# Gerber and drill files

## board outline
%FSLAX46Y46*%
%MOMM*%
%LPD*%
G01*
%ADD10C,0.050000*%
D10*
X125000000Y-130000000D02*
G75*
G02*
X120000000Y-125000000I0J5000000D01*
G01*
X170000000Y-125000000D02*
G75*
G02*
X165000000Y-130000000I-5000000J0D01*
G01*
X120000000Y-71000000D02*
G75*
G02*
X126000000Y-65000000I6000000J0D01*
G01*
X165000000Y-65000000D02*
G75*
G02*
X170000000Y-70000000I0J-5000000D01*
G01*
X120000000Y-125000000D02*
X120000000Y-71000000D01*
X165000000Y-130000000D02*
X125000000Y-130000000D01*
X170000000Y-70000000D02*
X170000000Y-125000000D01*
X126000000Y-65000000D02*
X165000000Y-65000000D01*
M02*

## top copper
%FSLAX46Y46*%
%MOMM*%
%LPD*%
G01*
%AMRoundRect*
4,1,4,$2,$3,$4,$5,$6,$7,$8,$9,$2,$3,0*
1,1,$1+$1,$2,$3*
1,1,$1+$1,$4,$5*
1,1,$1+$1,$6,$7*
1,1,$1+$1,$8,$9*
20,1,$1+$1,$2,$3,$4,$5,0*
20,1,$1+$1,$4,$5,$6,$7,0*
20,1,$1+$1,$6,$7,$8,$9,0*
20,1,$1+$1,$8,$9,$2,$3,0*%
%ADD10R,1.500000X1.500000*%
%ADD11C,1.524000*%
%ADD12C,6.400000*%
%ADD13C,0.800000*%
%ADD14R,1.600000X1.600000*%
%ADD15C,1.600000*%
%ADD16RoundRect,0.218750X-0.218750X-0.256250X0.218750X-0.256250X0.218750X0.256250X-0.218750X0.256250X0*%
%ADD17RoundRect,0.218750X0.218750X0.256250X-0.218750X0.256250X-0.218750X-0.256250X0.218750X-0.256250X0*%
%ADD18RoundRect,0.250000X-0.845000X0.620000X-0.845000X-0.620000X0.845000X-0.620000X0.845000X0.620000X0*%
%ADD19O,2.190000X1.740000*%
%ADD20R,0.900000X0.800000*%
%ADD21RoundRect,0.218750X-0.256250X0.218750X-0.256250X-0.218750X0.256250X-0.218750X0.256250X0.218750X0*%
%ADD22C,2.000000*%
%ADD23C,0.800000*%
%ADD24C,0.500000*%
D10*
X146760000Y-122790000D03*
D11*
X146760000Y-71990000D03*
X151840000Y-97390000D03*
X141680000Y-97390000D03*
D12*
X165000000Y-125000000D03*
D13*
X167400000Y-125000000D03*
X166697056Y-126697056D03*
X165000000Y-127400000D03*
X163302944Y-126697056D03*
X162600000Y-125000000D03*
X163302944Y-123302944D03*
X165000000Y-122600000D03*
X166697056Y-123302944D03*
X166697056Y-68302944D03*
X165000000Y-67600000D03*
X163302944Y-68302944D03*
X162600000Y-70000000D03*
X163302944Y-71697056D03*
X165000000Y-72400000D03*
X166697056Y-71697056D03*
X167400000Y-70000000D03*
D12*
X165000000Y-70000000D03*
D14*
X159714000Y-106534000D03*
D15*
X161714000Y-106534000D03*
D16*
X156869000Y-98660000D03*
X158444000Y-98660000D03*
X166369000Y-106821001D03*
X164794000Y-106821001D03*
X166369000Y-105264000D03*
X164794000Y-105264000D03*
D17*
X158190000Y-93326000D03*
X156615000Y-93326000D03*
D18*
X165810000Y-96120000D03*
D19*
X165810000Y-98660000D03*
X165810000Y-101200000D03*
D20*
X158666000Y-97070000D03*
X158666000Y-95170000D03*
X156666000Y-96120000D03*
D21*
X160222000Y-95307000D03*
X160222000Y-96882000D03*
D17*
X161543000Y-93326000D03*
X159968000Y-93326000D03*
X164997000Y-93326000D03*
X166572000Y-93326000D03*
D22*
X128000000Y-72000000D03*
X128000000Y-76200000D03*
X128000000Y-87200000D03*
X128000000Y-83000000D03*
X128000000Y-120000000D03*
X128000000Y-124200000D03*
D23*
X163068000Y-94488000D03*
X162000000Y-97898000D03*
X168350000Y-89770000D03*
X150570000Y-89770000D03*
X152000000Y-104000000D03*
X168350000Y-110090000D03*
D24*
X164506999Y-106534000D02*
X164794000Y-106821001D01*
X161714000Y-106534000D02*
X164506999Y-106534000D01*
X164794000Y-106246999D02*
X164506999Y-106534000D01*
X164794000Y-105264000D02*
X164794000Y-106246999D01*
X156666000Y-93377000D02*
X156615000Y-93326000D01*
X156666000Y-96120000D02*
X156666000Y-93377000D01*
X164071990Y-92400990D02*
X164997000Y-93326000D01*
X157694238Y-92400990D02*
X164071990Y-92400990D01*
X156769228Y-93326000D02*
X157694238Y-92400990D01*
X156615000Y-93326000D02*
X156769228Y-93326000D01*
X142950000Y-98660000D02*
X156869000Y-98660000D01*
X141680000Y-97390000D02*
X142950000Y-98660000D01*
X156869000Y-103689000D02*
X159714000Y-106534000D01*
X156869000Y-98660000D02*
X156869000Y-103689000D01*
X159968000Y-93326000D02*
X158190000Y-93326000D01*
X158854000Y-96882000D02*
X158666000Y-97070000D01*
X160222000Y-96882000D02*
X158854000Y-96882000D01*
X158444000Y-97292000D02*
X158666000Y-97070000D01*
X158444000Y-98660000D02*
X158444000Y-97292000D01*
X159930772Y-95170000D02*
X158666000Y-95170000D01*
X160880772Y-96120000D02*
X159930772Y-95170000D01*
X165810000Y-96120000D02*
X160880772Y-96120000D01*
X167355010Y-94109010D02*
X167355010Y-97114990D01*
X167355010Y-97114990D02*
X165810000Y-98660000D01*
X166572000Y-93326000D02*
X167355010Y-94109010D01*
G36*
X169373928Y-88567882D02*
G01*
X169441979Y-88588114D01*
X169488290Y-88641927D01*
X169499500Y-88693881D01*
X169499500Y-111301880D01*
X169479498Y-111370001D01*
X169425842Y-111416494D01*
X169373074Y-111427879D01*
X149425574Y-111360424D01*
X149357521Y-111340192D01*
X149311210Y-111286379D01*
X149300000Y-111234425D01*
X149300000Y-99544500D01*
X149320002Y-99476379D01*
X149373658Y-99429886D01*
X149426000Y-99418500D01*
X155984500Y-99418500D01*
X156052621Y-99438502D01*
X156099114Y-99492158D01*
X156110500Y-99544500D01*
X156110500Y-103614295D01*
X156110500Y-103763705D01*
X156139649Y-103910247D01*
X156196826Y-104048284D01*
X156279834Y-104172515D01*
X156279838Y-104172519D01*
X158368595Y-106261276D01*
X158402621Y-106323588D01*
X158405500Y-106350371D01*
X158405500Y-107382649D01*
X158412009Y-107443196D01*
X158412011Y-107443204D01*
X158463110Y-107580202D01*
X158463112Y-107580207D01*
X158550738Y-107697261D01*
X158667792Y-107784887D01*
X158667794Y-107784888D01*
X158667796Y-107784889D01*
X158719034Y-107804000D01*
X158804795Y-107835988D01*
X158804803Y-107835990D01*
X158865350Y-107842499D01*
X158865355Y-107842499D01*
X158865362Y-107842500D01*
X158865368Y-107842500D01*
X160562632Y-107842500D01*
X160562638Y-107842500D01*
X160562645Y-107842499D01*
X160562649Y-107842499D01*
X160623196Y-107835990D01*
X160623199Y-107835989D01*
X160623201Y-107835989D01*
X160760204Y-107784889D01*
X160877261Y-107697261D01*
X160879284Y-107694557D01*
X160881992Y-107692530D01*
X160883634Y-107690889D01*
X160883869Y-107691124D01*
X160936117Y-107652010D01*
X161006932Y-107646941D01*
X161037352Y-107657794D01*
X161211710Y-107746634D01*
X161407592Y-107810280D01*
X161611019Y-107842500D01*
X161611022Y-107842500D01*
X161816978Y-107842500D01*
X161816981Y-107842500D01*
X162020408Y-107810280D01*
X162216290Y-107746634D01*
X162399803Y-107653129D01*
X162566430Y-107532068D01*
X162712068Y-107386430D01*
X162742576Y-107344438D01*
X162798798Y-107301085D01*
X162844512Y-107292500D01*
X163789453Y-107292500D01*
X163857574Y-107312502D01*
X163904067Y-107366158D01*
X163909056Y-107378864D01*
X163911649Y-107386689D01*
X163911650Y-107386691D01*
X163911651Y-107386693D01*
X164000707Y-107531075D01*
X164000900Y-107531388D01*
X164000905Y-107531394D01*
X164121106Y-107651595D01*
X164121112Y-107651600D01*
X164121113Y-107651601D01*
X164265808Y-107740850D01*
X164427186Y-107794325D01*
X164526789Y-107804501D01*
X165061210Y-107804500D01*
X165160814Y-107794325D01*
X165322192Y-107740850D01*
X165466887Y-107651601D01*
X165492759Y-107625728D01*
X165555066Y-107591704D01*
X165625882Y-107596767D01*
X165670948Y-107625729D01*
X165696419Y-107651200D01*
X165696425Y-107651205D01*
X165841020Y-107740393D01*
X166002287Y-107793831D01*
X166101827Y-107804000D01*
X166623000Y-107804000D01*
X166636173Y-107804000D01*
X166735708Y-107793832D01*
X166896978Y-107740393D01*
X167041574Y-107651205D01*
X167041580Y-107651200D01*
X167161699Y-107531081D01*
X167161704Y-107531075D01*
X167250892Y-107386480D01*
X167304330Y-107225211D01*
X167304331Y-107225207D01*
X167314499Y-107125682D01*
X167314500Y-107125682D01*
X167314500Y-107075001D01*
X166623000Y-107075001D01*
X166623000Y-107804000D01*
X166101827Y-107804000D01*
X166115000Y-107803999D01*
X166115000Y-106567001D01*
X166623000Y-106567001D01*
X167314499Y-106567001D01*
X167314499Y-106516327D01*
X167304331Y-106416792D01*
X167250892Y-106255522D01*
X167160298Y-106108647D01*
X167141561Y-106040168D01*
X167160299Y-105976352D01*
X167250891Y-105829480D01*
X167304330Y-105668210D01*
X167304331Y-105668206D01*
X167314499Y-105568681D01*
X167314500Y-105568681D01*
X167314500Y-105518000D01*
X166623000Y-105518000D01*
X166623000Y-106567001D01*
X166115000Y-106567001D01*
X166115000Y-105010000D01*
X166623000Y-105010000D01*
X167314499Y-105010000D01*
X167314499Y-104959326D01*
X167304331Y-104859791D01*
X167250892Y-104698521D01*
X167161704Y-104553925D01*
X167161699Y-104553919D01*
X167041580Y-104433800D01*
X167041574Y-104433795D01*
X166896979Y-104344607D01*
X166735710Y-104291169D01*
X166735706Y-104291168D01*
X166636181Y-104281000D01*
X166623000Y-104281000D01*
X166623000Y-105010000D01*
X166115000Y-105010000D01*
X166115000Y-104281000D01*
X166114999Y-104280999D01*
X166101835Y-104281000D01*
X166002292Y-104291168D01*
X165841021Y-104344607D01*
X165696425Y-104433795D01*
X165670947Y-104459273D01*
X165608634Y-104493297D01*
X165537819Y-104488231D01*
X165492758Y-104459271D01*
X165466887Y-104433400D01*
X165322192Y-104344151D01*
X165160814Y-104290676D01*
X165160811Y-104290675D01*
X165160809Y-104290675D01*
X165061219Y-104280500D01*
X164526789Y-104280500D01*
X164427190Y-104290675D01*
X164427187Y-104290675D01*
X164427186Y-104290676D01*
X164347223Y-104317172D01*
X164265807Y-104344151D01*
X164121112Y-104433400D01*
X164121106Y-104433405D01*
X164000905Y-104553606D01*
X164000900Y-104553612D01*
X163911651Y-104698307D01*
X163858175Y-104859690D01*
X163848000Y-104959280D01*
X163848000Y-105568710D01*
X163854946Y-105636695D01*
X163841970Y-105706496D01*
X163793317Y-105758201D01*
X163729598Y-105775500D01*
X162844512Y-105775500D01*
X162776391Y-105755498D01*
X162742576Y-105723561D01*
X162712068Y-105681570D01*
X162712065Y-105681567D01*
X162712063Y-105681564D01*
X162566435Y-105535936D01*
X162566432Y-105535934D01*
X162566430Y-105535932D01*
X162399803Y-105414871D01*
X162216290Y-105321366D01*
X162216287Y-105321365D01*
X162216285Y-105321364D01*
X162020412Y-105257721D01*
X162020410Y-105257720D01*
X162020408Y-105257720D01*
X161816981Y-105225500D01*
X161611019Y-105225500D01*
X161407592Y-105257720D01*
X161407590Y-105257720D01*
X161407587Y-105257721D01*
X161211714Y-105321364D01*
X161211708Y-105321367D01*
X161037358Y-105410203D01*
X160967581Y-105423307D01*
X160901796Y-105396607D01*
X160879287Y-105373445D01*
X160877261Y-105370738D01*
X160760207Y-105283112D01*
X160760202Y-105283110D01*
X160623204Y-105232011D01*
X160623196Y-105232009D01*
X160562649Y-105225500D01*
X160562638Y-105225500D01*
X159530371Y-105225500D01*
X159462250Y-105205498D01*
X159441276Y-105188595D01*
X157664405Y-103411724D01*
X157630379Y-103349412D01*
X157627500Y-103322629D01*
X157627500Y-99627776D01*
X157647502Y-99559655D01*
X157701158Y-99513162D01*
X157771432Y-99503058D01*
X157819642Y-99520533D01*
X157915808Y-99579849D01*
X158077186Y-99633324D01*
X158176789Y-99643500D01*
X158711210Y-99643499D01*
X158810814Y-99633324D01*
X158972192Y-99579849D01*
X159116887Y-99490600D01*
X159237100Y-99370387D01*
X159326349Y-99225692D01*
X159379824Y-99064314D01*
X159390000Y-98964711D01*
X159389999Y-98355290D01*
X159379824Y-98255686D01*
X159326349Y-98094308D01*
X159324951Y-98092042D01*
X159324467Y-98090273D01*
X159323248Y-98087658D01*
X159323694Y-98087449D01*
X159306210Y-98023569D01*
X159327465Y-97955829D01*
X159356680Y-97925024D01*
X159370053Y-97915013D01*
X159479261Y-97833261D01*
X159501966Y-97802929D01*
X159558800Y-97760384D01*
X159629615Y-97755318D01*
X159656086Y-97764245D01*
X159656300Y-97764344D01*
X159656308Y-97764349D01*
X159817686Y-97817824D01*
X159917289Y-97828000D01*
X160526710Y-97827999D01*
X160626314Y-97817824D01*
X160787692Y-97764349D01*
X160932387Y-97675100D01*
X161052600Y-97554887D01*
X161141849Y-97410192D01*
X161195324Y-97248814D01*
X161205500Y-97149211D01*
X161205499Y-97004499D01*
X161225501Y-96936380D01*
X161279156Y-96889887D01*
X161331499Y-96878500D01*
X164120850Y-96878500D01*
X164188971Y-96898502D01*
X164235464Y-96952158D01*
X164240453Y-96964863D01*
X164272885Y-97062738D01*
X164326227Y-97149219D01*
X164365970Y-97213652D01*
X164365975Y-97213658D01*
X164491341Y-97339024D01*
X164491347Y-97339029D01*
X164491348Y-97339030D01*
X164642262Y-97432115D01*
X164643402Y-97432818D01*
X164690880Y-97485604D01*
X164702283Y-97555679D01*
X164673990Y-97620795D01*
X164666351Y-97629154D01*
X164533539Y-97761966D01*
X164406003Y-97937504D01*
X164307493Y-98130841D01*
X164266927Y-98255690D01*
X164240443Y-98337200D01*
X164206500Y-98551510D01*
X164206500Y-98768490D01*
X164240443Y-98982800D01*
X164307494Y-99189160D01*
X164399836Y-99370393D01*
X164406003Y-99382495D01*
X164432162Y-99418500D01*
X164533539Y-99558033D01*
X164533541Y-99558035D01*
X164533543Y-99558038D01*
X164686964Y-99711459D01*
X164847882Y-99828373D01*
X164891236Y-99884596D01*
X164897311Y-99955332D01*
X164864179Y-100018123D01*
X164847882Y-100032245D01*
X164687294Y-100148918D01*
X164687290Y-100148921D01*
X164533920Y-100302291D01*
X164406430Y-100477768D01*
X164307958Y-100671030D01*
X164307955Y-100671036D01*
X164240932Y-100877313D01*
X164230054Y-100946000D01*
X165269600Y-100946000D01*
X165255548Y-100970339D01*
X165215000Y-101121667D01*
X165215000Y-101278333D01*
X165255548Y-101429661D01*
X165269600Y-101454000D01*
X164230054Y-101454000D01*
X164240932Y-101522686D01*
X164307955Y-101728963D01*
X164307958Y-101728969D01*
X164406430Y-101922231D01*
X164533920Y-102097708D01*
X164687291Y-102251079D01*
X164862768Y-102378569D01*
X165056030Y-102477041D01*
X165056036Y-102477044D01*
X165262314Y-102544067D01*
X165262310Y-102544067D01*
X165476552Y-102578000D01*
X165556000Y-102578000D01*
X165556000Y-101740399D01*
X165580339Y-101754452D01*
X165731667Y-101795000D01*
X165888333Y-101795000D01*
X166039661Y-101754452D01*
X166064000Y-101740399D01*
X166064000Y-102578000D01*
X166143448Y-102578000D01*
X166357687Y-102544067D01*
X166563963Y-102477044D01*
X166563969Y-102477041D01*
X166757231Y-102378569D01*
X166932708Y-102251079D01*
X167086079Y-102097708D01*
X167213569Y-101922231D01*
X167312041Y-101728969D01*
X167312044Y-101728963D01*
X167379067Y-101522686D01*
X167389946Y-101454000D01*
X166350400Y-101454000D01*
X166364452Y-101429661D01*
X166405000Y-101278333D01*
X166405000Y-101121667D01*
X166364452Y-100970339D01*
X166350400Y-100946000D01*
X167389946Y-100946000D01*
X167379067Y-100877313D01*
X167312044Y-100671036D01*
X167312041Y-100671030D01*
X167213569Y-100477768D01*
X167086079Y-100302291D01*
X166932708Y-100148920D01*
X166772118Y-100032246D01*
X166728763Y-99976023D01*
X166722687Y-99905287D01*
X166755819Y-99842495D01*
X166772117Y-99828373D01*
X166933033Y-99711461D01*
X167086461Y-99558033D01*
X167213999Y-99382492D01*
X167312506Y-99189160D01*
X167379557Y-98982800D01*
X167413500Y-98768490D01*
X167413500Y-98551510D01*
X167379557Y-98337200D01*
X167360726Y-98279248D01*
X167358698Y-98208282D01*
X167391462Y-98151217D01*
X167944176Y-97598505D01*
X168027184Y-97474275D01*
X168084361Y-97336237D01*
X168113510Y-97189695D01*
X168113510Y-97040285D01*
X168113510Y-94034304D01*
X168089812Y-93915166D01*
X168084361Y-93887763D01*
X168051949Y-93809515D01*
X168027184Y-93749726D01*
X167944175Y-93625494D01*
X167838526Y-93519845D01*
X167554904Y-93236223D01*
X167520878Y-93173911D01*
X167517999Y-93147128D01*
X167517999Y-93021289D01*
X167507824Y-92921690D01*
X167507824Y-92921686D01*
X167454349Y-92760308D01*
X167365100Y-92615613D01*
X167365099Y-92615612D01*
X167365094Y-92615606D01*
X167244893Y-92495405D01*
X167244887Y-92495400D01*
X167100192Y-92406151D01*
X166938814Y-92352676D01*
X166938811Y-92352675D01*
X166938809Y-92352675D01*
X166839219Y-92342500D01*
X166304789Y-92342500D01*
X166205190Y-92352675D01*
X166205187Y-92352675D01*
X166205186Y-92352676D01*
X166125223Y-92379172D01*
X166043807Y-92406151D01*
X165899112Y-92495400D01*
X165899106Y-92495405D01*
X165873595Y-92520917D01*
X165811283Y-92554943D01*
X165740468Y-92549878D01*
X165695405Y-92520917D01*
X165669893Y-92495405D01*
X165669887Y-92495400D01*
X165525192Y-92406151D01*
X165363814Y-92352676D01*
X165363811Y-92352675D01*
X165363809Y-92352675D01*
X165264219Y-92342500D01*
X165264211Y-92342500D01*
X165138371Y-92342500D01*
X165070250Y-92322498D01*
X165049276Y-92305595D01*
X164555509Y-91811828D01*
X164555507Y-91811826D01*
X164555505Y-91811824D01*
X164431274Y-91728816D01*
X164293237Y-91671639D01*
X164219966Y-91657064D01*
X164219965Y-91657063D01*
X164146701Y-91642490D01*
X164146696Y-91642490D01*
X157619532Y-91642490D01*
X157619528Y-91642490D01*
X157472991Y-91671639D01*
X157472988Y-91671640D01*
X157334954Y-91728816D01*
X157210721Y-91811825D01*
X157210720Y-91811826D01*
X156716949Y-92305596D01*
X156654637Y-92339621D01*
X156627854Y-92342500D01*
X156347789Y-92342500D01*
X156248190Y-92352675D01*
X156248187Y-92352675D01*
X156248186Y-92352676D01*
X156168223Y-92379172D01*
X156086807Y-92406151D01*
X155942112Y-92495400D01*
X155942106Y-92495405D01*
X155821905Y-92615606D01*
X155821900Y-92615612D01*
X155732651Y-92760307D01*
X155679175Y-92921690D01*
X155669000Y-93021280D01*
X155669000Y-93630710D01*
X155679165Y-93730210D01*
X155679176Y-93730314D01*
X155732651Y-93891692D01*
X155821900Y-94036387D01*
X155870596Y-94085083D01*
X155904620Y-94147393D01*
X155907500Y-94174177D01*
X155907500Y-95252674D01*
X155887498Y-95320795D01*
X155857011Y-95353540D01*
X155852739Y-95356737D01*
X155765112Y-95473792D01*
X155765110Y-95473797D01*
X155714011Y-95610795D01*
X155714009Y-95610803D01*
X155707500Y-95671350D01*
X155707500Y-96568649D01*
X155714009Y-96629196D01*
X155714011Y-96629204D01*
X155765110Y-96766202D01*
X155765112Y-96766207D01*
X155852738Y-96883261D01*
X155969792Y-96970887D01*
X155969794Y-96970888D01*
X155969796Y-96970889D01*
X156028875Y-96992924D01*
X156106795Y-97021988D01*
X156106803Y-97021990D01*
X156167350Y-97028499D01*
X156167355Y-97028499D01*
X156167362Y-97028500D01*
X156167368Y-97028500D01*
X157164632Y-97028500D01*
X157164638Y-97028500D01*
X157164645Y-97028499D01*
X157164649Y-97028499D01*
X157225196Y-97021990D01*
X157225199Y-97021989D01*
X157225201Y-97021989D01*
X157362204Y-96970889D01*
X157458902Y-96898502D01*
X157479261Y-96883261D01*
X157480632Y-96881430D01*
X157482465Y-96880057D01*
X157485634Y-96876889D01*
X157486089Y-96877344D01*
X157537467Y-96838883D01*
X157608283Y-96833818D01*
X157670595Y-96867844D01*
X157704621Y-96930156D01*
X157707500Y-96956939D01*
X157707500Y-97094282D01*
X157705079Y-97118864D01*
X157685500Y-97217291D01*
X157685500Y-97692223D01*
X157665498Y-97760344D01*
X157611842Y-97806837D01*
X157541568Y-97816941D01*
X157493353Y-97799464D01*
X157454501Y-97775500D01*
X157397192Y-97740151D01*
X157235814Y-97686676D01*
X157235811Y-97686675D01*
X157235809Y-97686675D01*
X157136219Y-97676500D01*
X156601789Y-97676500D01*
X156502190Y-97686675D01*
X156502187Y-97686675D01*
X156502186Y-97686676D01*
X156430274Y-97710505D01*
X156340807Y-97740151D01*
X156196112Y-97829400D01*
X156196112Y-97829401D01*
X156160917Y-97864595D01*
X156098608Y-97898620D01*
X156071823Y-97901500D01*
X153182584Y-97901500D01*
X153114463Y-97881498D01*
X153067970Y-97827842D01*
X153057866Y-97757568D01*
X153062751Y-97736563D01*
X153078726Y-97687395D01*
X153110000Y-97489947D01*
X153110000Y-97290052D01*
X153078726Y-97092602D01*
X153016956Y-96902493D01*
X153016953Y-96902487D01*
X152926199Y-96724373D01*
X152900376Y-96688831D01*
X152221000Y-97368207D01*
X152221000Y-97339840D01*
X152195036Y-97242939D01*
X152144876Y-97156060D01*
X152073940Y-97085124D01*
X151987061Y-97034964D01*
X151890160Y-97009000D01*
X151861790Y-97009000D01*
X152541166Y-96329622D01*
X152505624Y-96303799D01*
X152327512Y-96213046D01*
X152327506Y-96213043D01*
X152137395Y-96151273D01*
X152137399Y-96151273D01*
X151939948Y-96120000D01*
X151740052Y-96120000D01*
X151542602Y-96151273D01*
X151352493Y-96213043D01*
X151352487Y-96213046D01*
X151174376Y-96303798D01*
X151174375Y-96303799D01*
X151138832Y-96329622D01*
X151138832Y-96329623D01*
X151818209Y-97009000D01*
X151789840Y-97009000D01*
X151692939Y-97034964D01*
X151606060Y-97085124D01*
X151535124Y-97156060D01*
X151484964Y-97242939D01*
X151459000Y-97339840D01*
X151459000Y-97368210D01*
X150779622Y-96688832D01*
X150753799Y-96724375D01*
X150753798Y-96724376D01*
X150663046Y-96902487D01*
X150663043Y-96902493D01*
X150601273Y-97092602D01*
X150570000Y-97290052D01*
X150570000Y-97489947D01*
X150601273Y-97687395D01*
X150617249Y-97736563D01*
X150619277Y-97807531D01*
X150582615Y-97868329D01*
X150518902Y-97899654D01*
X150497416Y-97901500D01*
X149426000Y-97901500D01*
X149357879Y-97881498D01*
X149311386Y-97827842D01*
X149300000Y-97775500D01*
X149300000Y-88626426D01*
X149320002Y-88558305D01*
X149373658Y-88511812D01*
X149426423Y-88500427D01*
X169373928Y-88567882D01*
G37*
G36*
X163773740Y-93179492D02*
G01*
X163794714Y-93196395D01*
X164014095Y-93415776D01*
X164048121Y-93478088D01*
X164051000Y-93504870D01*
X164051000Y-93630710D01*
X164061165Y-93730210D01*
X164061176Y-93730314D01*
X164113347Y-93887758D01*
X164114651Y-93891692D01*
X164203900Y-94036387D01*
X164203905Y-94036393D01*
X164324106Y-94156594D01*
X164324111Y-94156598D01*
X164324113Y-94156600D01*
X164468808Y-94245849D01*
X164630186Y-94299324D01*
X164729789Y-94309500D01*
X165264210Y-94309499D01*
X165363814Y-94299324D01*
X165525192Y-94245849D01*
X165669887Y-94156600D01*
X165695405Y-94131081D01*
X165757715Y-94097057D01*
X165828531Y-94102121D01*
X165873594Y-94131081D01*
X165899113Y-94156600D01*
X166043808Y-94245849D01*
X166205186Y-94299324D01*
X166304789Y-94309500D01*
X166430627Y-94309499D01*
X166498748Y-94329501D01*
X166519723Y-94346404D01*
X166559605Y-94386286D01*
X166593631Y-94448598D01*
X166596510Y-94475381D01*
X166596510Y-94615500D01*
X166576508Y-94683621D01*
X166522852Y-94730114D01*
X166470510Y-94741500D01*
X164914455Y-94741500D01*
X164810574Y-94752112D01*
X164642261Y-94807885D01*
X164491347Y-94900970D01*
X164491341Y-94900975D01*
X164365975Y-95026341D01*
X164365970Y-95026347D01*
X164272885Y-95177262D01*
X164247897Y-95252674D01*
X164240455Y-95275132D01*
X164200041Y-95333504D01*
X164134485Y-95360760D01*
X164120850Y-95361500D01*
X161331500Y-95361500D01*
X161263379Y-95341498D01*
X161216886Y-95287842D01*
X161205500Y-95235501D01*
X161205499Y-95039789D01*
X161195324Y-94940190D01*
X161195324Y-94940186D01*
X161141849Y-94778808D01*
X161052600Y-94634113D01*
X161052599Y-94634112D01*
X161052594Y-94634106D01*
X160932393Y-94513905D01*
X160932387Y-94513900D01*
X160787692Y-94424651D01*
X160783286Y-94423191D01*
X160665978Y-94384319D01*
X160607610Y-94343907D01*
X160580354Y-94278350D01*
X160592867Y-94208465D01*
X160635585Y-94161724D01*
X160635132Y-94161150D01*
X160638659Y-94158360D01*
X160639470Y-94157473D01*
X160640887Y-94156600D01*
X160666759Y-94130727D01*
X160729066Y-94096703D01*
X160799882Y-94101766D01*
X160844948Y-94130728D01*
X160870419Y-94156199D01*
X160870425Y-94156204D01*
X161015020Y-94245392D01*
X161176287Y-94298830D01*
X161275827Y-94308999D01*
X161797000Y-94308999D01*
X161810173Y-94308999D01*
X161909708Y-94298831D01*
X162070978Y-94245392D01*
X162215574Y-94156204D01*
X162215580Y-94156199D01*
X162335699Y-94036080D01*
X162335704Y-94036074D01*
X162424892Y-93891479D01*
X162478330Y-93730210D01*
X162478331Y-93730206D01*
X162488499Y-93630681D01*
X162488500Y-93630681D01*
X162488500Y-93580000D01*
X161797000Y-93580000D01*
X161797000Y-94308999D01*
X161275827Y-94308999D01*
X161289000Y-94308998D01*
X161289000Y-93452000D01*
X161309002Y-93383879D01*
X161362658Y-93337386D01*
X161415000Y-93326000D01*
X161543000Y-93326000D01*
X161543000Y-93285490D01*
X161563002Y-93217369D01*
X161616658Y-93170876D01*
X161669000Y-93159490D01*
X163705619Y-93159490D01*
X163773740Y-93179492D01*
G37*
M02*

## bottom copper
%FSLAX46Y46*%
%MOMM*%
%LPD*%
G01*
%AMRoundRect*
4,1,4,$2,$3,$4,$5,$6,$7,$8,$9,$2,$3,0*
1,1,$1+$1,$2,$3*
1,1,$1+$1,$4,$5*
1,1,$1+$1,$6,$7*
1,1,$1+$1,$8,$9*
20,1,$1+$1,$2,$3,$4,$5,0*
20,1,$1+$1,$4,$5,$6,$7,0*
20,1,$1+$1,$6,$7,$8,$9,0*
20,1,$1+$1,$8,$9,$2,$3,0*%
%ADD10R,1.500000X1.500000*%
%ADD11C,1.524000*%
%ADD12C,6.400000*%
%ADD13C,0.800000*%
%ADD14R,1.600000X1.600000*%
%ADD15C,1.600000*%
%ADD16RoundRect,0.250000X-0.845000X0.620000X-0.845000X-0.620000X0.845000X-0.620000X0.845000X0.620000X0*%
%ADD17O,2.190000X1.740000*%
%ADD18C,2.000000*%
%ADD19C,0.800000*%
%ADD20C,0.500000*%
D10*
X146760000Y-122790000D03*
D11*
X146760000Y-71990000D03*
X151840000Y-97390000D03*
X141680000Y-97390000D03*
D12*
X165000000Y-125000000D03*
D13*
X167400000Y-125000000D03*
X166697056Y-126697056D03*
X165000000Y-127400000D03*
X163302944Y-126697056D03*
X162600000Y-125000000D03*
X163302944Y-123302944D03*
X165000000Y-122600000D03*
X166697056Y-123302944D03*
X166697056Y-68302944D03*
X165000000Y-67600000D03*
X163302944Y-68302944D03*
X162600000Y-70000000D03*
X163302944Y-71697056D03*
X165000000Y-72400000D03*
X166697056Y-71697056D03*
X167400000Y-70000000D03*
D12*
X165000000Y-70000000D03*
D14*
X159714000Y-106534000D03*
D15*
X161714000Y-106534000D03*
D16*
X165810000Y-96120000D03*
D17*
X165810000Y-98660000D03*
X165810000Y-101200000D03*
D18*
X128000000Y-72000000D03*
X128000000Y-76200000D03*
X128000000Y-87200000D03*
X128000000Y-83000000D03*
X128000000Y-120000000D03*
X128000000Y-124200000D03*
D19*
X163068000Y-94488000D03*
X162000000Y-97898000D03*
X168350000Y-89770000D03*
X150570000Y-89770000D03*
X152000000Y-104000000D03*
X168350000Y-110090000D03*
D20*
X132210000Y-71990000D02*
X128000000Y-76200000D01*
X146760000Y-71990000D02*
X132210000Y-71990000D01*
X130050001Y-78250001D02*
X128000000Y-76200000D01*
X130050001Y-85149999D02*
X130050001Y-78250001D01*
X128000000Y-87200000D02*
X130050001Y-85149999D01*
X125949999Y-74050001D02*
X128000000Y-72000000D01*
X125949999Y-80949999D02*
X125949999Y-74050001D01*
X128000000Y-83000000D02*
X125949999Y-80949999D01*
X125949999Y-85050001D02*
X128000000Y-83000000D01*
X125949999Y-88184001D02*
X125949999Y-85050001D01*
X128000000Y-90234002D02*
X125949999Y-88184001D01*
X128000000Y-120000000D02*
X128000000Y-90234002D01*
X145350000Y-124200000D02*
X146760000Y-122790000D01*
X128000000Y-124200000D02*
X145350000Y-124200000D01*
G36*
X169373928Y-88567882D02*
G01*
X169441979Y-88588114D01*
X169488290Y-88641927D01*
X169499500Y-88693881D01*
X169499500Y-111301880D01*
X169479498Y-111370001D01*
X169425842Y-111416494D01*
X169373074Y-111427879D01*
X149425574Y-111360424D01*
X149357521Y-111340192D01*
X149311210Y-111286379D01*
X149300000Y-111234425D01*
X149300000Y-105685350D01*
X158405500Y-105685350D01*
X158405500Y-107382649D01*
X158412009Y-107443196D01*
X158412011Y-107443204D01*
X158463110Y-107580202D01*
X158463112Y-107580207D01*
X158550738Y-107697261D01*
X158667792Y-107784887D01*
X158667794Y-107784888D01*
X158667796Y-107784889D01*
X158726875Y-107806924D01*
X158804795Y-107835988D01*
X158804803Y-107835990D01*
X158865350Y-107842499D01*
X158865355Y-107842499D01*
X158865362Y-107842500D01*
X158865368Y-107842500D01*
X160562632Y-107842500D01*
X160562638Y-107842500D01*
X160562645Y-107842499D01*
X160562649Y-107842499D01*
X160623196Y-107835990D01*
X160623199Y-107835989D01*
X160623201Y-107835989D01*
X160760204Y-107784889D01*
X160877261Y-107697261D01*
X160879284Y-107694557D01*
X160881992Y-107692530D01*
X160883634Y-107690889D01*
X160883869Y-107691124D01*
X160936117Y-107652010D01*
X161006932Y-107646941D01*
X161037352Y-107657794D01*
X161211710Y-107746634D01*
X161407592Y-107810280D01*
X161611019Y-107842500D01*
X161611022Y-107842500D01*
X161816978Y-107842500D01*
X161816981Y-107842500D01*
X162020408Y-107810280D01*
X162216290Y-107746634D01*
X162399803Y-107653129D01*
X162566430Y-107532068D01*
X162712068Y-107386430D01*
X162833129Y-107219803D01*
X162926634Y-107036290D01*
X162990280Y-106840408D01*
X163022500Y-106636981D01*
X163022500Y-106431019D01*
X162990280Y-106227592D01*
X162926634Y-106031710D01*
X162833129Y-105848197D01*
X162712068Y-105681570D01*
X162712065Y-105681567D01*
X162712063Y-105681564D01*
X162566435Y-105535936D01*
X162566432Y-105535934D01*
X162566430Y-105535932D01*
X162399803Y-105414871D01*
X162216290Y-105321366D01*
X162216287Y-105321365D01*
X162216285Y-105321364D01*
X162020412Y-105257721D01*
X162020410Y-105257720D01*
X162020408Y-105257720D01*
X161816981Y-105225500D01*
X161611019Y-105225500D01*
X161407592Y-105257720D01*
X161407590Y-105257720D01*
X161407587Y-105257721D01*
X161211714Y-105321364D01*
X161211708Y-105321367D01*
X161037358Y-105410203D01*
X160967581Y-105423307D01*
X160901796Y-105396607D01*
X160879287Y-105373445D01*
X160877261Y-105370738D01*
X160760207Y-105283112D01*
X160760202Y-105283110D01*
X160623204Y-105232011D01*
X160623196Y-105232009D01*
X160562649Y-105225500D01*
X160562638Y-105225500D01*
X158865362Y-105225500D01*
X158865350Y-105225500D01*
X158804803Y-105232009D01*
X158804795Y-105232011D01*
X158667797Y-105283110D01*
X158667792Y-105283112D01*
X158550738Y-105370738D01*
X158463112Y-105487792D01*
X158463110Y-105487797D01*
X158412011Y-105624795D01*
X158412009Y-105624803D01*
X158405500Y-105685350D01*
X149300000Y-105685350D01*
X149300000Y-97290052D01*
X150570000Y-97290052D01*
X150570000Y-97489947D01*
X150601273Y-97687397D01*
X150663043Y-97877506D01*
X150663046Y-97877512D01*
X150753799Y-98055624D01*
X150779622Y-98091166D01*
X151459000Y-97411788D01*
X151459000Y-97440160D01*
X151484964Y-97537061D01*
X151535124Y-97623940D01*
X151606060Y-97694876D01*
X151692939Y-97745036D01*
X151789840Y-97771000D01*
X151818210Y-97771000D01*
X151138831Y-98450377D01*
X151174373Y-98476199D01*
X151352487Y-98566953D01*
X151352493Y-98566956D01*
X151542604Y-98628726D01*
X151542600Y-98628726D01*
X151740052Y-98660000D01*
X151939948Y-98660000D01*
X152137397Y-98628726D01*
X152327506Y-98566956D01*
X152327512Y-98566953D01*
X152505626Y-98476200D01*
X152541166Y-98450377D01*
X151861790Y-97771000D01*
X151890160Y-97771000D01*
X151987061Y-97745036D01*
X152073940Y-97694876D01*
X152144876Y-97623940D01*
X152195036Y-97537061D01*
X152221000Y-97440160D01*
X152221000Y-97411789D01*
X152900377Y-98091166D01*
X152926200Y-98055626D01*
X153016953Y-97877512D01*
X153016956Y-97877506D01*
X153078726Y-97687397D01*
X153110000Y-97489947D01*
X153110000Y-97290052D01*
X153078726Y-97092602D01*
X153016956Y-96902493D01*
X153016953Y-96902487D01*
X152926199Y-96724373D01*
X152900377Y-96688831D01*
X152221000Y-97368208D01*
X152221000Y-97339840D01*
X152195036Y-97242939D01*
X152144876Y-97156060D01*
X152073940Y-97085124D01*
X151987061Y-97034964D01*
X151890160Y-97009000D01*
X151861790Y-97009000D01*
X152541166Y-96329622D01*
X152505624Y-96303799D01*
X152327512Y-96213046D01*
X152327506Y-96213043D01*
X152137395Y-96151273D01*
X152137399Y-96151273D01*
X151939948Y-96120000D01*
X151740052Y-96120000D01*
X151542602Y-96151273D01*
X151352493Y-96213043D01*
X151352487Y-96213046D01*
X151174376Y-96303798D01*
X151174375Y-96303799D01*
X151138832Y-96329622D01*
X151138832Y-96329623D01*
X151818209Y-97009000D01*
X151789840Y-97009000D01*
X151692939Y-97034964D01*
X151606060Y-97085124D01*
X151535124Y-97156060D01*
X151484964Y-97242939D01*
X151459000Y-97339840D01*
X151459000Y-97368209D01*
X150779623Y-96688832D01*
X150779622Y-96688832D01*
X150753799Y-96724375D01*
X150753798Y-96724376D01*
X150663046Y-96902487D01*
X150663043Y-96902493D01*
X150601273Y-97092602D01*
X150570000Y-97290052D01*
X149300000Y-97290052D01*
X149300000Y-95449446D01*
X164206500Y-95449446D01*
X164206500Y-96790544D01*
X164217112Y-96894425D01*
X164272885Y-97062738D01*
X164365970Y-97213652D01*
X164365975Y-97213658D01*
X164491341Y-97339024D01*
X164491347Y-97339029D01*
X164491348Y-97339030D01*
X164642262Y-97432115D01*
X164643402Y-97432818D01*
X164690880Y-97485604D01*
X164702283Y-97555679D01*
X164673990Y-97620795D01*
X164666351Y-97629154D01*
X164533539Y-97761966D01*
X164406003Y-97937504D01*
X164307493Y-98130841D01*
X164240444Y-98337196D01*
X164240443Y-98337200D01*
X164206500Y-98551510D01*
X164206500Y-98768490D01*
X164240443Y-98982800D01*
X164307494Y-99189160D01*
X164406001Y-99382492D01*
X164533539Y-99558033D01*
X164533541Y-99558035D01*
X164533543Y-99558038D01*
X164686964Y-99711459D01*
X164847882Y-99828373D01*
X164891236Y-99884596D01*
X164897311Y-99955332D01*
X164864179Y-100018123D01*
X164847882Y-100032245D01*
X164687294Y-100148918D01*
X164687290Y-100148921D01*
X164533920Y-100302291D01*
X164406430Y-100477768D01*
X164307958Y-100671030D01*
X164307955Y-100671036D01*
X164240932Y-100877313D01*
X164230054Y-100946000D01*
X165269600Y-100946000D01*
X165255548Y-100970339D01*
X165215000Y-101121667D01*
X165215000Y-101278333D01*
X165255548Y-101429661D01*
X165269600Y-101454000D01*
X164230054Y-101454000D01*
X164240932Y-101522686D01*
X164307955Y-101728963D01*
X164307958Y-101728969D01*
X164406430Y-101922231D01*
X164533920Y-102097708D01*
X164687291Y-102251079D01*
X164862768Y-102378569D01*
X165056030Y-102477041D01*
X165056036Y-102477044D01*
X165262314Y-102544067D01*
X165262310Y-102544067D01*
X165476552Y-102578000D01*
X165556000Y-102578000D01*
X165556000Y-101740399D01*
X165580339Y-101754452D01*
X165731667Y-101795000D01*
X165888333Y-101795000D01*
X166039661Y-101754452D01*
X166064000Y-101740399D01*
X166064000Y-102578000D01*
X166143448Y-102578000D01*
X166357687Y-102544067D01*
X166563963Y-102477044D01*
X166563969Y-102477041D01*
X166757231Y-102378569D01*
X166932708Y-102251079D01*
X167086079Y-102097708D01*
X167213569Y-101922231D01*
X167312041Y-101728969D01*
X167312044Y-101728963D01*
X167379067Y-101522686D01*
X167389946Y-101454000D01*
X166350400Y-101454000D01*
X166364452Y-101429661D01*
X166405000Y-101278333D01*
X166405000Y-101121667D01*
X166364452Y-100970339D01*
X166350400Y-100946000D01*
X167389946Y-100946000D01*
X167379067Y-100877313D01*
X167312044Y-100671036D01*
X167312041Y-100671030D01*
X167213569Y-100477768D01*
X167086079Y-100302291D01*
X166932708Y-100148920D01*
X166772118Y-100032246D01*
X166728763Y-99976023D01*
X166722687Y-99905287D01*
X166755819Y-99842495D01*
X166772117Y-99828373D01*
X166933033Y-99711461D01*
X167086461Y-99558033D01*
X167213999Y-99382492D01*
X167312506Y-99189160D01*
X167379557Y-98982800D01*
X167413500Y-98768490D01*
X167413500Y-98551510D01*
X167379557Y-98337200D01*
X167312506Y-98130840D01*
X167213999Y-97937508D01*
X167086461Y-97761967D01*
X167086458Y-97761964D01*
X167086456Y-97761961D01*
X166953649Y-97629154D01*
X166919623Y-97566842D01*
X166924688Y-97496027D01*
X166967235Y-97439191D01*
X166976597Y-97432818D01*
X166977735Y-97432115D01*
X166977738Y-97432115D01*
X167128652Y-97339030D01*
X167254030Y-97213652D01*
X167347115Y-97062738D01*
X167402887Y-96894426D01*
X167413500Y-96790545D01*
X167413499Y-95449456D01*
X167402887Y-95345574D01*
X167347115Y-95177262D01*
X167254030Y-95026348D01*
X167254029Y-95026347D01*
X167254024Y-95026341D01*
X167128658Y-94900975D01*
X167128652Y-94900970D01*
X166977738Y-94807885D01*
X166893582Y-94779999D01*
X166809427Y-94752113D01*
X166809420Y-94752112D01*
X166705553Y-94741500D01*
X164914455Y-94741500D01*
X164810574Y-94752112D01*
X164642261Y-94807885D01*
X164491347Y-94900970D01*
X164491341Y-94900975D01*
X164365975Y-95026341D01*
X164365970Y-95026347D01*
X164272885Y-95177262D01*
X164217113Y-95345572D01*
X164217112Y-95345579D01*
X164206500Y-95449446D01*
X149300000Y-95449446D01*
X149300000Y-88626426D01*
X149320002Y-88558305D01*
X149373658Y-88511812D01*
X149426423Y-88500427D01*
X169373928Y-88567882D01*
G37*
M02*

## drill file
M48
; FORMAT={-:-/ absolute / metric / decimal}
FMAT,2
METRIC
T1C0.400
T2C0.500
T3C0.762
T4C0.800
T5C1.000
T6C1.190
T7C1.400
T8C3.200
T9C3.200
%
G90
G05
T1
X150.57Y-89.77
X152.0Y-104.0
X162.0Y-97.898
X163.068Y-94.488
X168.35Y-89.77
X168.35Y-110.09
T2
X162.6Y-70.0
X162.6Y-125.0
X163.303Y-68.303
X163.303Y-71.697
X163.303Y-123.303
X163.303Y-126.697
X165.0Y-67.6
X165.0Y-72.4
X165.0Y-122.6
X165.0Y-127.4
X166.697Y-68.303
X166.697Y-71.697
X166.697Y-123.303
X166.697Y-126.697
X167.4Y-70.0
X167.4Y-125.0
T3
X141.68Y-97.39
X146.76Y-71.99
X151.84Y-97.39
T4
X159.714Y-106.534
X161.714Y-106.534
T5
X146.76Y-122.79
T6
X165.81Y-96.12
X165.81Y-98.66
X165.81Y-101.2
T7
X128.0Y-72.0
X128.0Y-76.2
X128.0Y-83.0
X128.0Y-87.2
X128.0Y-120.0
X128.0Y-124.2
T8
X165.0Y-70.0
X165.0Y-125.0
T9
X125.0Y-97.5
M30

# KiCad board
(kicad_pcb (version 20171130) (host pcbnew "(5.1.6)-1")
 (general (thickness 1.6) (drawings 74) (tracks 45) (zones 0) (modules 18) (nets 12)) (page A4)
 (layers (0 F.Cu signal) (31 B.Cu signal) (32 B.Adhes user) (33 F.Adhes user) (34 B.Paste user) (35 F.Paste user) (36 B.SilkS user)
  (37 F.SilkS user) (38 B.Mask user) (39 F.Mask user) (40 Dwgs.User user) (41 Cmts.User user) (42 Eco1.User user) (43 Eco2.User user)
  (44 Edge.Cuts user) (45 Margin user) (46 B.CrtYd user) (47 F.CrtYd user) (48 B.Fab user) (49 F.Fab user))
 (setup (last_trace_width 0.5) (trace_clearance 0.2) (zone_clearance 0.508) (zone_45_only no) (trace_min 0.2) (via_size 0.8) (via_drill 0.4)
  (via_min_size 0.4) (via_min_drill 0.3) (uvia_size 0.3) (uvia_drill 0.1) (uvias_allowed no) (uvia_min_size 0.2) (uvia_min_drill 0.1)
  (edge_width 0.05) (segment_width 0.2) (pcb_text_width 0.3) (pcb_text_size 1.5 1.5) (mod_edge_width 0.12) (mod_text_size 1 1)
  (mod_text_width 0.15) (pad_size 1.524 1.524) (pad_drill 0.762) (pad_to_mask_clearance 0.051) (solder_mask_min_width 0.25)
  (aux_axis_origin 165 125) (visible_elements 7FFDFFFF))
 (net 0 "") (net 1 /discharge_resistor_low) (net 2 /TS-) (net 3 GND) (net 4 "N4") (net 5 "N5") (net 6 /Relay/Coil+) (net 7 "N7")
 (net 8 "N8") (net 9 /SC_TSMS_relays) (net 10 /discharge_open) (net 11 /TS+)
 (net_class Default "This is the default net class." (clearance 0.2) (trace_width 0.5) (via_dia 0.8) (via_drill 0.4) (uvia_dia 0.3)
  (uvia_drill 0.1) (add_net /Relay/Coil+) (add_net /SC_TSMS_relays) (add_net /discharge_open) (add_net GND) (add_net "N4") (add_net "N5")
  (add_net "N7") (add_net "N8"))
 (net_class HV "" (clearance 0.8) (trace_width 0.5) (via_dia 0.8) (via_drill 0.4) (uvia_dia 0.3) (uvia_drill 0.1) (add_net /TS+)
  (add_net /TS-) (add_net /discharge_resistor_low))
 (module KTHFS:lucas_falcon (layer F.Cu) (at 165 79)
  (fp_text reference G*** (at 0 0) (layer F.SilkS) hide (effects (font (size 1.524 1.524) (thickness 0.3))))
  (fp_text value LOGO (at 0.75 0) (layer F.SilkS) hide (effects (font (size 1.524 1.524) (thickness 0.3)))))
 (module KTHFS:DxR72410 (layer F.Cu) (at 146.76 122.79 90)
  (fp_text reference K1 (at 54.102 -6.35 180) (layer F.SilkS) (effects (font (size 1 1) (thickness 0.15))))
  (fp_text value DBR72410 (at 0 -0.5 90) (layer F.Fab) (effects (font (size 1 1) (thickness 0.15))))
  (pad 1 thru_hole rect (at 0 0 90) (size 1.5 1.5) (drill 1) (layers *.Cu *.Mask) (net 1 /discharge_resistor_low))
  (pad 2 thru_hole circle (at 50.8 0 90) (size 1.524 1.524) (drill 0.762) (layers *.Cu *.Mask) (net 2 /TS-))
  (pad 3 thru_hole circle (at 25.4 5.08 90) (size 1.524 1.524) (drill 0.762) (layers *.Cu *.Mask) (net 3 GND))
  (pad 4 thru_hole circle (at 25.4 -5.08 90) (size 1.524 1.524) (drill 0.762) (layers *.Cu *.Mask) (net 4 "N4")))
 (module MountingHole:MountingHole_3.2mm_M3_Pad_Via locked (layer F.Cu) (at 165 125)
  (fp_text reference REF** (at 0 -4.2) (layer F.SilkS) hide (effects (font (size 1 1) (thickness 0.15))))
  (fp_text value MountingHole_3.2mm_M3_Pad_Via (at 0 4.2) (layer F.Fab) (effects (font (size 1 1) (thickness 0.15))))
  (pad 1 thru_hole circle (at 0 0) (size 6.4 6.4) (drill 3.2) (layers *.Cu *.Mask))
  (pad 1 thru_hole circle (at 2.4 0) (size 0.8 0.8) (drill 0.5) (layers *.Cu *.Mask))
  (pad 1 thru_hole circle (at 1.697056 1.697056) (size 0.8 0.8) (drill 0.5) (layers *.Cu *.Mask))
  (pad 1 thru_hole circle (at 0 2.4) (size 0.8 0.8) (drill 0.5) (layers *.Cu *.Mask))
  (pad 1 thru_hole circle (at -1.697056 1.697056) (size 0.8 0.8) (drill 0.5) (layers *.Cu *.Mask))
  (pad 1 thru_hole circle (at -2.4 0) (size 0.8 0.8) (drill 0.5) (layers *.Cu *.Mask))
  (pad 1 thru_hole circle (at -1.697056 -1.697056) (size 0.8 0.8) (drill 0.5) (layers *.Cu *.Mask))
  (pad 1 thru_hole circle (at 0 -2.4) (size 0.8 0.8) (drill 0.5) (layers *.Cu *.Mask))
  (pad 1 thru_hole circle (at 1.697056 -1.697056) (size 0.8 0.8) (drill 0.5) (layers *.Cu *.Mask)))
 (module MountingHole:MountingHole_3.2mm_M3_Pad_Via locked (layer F.Cu) (at 165 70)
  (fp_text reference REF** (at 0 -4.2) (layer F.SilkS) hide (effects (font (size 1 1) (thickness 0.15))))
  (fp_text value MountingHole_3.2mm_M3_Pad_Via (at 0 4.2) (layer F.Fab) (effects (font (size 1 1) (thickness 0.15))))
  (pad 1 thru_hole circle (at 1.697056 -1.697056) (size 0.8 0.8) (drill 0.5) (layers *.Cu *.Mask))
  (pad 1 thru_hole circle (at 0 -2.4) (size 0.8 0.8) (drill 0.5) (layers *.Cu *.Mask))
  (pad 1 thru_hole circle (at -1.697056 -1.697056) (size 0.8 0.8) (drill 0.5) (layers *.Cu *.Mask))
  (pad 1 thru_hole circle (at -2.4 0) (size 0.8 0.8) (drill 0.5) (layers *.Cu *.Mask))
  (pad 1 thru_hole circle (at -1.697056 1.697056) (size 0.8 0.8) (drill 0.5) (layers *.Cu *.Mask))
  (pad 1 thru_hole circle (at 0 2.4) (size 0.8 0.8) (drill 0.5) (layers *.Cu *.Mask))
  (pad 1 thru_hole circle (at 1.697056 1.697056) (size 0.8 0.8) (drill 0.5) (layers *.Cu *.Mask))
  (pad 1 thru_hole circle (at 2.4 0) (size 0.8 0.8) (drill 0.5) (layers *.Cu *.Mask))
  (pad 1 thru_hole circle (at 0 0) (size 6.4 6.4) (drill 3.2) (layers *.Cu *.Mask)))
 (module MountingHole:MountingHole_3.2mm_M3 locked (layer F.Cu) (at 125 97.5)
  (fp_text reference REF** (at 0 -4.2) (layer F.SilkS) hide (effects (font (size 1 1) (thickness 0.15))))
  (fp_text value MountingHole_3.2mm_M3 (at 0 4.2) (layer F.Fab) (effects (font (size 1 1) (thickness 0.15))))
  (pad 1 np_thru_hole circle (at 0 0) (size 3.2 3.2) (drill 3.2) (layers *.Cu *.Mask)))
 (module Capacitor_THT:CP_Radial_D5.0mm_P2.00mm (layer F.Cu) (at 159.714 106.534)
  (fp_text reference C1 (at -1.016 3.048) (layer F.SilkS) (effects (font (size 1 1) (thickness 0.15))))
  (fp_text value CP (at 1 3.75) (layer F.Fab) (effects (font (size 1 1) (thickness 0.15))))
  (pad 1 thru_hole rect (at 0 0) (size 1.6 1.6) (drill 0.8) (layers *.Cu *.Mask) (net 4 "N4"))
  (pad 2 thru_hole circle (at 2 0) (size 1.6 1.6) (drill 0.8) (layers *.Cu *.Mask) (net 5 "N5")))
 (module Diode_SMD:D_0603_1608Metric (layer F.Cu) (at 157.6565 98.66)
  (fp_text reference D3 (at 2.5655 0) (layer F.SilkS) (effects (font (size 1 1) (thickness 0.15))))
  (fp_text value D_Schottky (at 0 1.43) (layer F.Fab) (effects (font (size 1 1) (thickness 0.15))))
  (pad 1 smd roundrect (at -0.7875 0) (size 0.875 0.95) (layers F.Cu F.Paste F.Mask) (roundrect_rratio 0.25) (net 4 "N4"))
  (pad 2 smd roundrect (at 0.7875 0) (size 0.875 0.95) (layers F.Cu F.Paste F.Mask) (roundrect_rratio 0.25) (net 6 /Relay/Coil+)))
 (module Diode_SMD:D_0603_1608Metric (layer F.Cu) (at 165.5815 106.821001)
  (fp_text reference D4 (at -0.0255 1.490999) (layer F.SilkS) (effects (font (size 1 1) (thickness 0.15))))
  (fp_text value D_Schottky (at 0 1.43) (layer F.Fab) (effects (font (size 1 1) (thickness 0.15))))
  (pad 2 smd roundrect (at 0.7875 0) (size 0.875 0.95) (layers F.Cu F.Paste F.Mask) (roundrect_rratio 0.25) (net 3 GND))
  (pad 1 smd roundrect (at -0.7875 0) (size 0.875 0.95) (layers F.Cu F.Paste F.Mask) (roundrect_rratio 0.25) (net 5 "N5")))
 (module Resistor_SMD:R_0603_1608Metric (layer F.Cu) (at 165.5815 105.264)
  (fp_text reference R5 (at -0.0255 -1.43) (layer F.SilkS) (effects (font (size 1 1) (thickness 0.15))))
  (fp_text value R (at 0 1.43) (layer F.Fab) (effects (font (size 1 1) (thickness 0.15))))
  (pad 2 smd roundrect (at 0.7875 0) (size 0.875 0.95) (layers F.Cu F.Paste F.Mask) (roundrect_rratio 0.25) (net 3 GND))
  (pad 1 smd roundrect (at -0.7875 0) (size 0.875 0.95) (layers F.Cu F.Paste F.Mask) (roundrect_rratio 0.25) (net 5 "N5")))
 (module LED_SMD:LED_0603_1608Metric (layer F.Cu) (at 157.4025 93.326 180)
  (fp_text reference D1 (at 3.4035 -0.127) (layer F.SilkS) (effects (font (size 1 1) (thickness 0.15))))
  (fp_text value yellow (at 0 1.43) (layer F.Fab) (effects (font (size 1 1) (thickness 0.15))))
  (pad 1 smd roundrect (at -0.7875 0 180) (size 0.875 0.95) (layers F.Cu F.Paste F.Mask) (roundrect_rratio 0.25) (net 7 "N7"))
  (pad 2 smd roundrect (at 0.7875 0 180) (size 0.875 0.95) (layers F.Cu F.Paste F.Mask) (roundrect_rratio 0.25) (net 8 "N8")))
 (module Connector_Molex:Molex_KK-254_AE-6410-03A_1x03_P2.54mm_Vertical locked (layer F.Cu) (at 165.81 96.12 270)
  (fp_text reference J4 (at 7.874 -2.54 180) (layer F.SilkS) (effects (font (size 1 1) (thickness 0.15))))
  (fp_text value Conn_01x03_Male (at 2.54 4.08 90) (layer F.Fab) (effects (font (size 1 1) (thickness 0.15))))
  (pad 1 thru_hole roundrect (at 0 0 270) (size 1.74 2.19) (drill 1.19) (layers *.Cu *.Mask) (roundrect_rratio 0.143678)
   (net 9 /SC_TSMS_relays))
  (pad 2 thru_hole oval (at 2.54 0 270) (size 1.74 2.19) (drill 1.19) (layers *.Cu *.Mask) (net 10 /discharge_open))
  (pad 3 thru_hole oval (at 5.08 0 270) (size 1.74 2.19) (drill 1.19) (layers *.Cu *.Mask) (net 3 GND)))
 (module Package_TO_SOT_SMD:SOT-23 (layer F.Cu) (at 157.666 96.12 180)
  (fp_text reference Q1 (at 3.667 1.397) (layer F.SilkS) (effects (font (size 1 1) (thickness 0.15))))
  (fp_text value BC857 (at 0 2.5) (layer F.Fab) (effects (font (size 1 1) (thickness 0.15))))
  (pad 1 smd rect (at -1 -0.95 180) (size 0.9 0.8) (layers F.Cu F.Paste F.Mask) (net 6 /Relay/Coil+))
  (pad 2 smd rect (at -1 0.95 180) (size 0.9 0.8) (layers F.Cu F.Paste F.Mask) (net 9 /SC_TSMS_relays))
  (pad 3 smd rect (at 1 0 180) (size 0.9 0.8) (layers F.Cu F.Paste F.Mask) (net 8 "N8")))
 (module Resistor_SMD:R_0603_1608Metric (layer F.Cu) (at 160.222 96.0945 270)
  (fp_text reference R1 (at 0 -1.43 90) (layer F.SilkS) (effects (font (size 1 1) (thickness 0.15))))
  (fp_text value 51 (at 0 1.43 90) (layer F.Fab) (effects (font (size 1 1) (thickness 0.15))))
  (pad 1 smd roundrect (at -0.7875 0 270) (size 0.875 0.95) (layers F.Cu F.Paste F.Mask) (roundrect_rratio 0.25) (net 9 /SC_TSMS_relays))
  (pad 2 smd roundrect (at 0.7875 0 270) (size 0.875 0.95) (layers F.Cu F.Paste F.Mask) (roundrect_rratio 0.25) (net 6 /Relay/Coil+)))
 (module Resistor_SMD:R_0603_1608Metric (layer F.Cu) (at 160.7555 93.326 180)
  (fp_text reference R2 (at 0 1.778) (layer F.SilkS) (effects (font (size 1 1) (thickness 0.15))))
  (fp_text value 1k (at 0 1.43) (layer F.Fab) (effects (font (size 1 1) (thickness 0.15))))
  (pad 1 smd roundrect (at -0.7875 0 180) (size 0.875 0.95) (layers F.Cu F.Paste F.Mask) (roundrect_rratio 0.25) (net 3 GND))
  (pad 2 smd roundrect (at 0.7875 0 180) (size 0.875 0.95) (layers F.Cu F.Paste F.Mask) (roundrect_rratio 0.25) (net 7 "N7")))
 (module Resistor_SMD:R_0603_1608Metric (layer F.Cu) (at 165.7845 93.326 180)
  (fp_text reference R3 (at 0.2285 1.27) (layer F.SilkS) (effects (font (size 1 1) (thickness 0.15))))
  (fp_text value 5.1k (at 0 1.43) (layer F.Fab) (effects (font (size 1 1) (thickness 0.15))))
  (pad 2 smd roundrect (at 0.7875 0 180) (size 0.875 0.95) (layers F.Cu F.Paste F.Mask) (roundrect_rratio 0.25) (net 8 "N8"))
  (pad 1 smd roundrect (at -0.7875 0 180) (size 0.875 0.95) (layers F.Cu F.Paste F.Mask) (roundrect_rratio 0.25) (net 10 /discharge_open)))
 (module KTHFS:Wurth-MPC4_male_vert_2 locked (layer F.Cu) (at 128 72 270)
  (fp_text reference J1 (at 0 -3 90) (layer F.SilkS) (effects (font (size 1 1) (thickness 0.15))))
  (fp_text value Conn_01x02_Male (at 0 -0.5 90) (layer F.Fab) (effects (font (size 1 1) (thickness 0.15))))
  (pad 1 thru_hole circle (at 0 0 270) (size 2 2) (drill 1.4) (layers *.Cu *.Mask) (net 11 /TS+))
  (pad 2 thru_hole circle (at 4.2 0 270) (size 2 2) (drill 1.4) (layers *.Cu *.Mask) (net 2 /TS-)))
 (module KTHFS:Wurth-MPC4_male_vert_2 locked (layer F.Cu) (at 128 83 270)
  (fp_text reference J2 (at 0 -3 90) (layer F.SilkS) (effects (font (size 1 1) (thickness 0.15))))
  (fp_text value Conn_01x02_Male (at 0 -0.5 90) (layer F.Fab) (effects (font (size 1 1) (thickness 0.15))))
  (pad 2 thru_hole circle (at 4.2 0 270) (size 2 2) (drill 1.4) (layers *.Cu *.Mask) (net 2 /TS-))
  (pad 1 thru_hole circle (at 0 0 270) (size 2 2) (drill 1.4) (layers *.Cu *.Mask) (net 11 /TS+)))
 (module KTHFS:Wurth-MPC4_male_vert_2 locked (layer F.Cu) (at 128 120 270)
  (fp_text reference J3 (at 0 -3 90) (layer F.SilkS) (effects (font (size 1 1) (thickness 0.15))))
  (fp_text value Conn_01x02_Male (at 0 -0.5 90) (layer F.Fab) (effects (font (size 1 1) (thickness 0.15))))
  (pad 1 thru_hole circle (at 0 0 270) (size 2 2) (drill 1.4) (layers *.Cu *.Mask) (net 11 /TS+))
  (pad 2 thru_hole circle (at 4.2 0 270) (size 2 2) (drill 1.4) (layers *.Cu *.Mask) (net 1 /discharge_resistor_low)))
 (gr_arc (start 125 125) (end 120 125) (angle -90) (layer Edge.Cuts) (width 0.05))
 (gr_arc (start 165 125) (end 165 130) (angle -90) (layer Edge.Cuts) (width 0.05))
 (gr_arc (start 126 71) (end 126 65) (angle -90) (layer Edge.Cuts) (width 0.05))
 (gr_arc (start 165 70) (end 170 70) (angle -90) (layer Edge.Cuts) (width 0.05))
 (gr_line (start 120 125) (end 120 71) (layer Edge.Cuts) (width 0.05))
 (gr_line (start 165 130) (end 125 130) (layer Edge.Cuts) (width 0.05))
 (gr_line (start 170 70) (end 170 125) (layer Edge.Cuts) (width 0.05))
 (gr_line (start 126 65) (end 165 65) (layer Edge.Cuts) (width 0.05))
 (segment (start 164.506999 106.534) (end 164.794 106.821001) (width 0.5) (layer F.Cu) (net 5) (status 30))
 (segment (start 161.714 106.534) (end 164.506999 106.534) (width 0.5) (layer F.Cu) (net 5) (status 30))
 (segment (start 164.794 106.246999) (end 164.506999 106.534) (width 0.5) (layer F.Cu) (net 5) (status 20))
 (segment (start 164.794 105.264) (end 164.794 106.246999) (width 0.5) (layer F.Cu) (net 5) (status 10))
 (segment (start 156.666 93.377) (end 156.615 93.326) (width 0.5) (layer F.Cu) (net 8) (status 30))
 (segment (start 156.666 96.12) (end 156.666 93.377) (width 0.5) (layer F.Cu) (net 8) (status 30))
 (segment (start 164.07199 92.40099) (end 164.997 93.326) (width 0.5) (layer F.Cu) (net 8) (status 20))
 (segment (start 157.694238 92.40099) (end 164.07199 92.40099) (width 0.5) (layer F.Cu) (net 8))
 (segment (start 156.769228 93.326) (end 157.694238 92.40099) (width 0.5) (layer F.Cu) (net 8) (status 10))
 (segment (start 156.615 93.326) (end 156.769228 93.326) (width 0.5) (layer F.Cu) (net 8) (status 30))
 (via (at 163.068 94.488) (size 0.8) (drill 0.4) (layers F.Cu B.Cu) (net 3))
 (via (at 162 97.898) (size 0.8) (drill 0.4) (layers F.Cu B.Cu) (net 3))
 (via (at 168.35 89.77) (size 0.8) (drill 0.4) (layers F.Cu B.Cu) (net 3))
 (via (at 150.57 89.77) (size 0.8) (drill 0.4) (layers F.Cu B.Cu) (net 3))
 (via (at 152 104) (size 0.8) (drill 0.4) (layers F.Cu B.Cu) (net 3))
 (via (at 168.35 110.09) (size 0.8) (drill 0.4) (layers F.Cu B.Cu) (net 3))
 (segment (start 132.21 71.99) (end 128 76.2) (width 0.5) (layer B.Cu) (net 2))
 (segment (start 146.76 71.99) (end 132.21 71.99) (width 0.5) (layer B.Cu) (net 2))
 (segment (start 130.050001 78.250001) (end 128 76.2) (width 0.5) (layer B.Cu) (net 2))
 (segment (start 130.050001 85.149999) (end 130.050001 78.250001) (width 0.5) (layer B.Cu) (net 2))
 (segment (start 128 87.2) (end 130.050001 85.149999) (width 0.5) (layer B.Cu) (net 2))
 (segment (start 125.949999 74.050001) (end 128 72) (width 0.5) (layer B.Cu) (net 11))
 (segment (start 125.949999 80.949999) (end 125.949999 74.050001) (width 0.5) (layer B.Cu) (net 11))
 (segment (start 128 83) (end 125.949999 80.949999) (width 0.5) (layer B.Cu) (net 11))
 (segment (start 125.949999 85.050001) (end 128 83) (width 0.5) (layer B.Cu) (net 11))
 (segment (start 125.949999 88.184001) (end 125.949999 85.050001) (width 0.5) (layer B.Cu) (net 11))
 (segment (start 128 90.234002) (end 125.949999 88.184001) (width 0.5) (layer B.Cu) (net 11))
 (segment (start 128 120) (end 128 90.234002) (width 0.5) (layer B.Cu) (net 11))
 (segment (start 142.95 98.66) (end 156.869 98.66) (width 0.5) (layer F.Cu) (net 4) (status 20))
 (segment (start 141.68 97.39) (end 142.95 98.66) (width 0.5) (layer F.Cu) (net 4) (status 10))
 (segment (start 156.869 103.689) (end 159.714 106.534) (width 0.5) (layer F.Cu) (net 4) (status 20))
 (segment (start 156.869 98.66) (end 156.869 103.689) (width 0.5) (layer F.Cu) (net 4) (status 10))
 (segment (start 159.968 93.326) (end 158.19 93.326) (width 0.5) (layer F.Cu) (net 7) (status 30))
 (segment (start 158.854 96.882) (end 158.666 97.07) (width 0.5) (layer F.Cu) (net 6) (status 30))
 (segment (start 160.222 96.882) (end 158.854 96.882) (width 0.5) (layer F.Cu) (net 6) (status 30))
 (segment (start 158.444 97.292) (end 158.666 97.07) (width 0.5) (layer F.Cu) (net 6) (status 30))
 (segment (start 158.444 98.66) (end 158.444 97.292) (width 0.5) (layer F.Cu) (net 6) (status 30))
 (segment (start 145.35 124.2) (end 146.76 122.79) (width 0.5) (layer B.Cu) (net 1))
 (segment (start 128 124.2) (end 145.35 124.2) (width 0.5) (layer B.Cu) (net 1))
 (segment (start 159.930772 95.17) (end 158.666 95.17) (width 0.5) (layer F.Cu) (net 9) (status 30))
 (segment (start 160.880772 96.12) (end 159.930772 95.17) (width 0.5) (layer F.Cu) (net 9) (status 20))
 (segment (start 165.81 96.12) (end 160.880772 96.12) (width 0.5) (layer F.Cu) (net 9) (status 10))
 (segment (start 167.35501 94.10901) (end 167.35501 97.11499) (width 0.5) (layer F.Cu) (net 10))
 (segment (start 167.35501 97.11499) (end 165.81 98.66) (width 0.5) (layer F.Cu) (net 10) (status 20))
 (segment (start 166.572 93.326) (end 167.35501 94.10901) (width 0.5) (layer F.Cu) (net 10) (status 10))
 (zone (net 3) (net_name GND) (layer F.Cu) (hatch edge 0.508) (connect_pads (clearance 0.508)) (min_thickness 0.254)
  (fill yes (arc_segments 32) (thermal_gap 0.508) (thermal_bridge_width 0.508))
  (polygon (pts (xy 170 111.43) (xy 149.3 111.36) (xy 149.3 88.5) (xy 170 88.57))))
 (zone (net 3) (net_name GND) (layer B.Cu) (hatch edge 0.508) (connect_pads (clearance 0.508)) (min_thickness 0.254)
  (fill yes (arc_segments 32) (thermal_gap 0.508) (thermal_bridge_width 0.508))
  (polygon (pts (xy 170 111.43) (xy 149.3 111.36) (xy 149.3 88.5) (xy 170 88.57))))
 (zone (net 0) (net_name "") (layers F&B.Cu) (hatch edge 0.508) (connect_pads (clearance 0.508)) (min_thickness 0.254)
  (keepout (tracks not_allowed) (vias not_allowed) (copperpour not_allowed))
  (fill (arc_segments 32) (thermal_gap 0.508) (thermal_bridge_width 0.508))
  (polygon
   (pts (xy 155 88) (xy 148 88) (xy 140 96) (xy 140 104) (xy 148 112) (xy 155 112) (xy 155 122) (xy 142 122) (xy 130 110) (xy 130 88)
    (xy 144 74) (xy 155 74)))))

